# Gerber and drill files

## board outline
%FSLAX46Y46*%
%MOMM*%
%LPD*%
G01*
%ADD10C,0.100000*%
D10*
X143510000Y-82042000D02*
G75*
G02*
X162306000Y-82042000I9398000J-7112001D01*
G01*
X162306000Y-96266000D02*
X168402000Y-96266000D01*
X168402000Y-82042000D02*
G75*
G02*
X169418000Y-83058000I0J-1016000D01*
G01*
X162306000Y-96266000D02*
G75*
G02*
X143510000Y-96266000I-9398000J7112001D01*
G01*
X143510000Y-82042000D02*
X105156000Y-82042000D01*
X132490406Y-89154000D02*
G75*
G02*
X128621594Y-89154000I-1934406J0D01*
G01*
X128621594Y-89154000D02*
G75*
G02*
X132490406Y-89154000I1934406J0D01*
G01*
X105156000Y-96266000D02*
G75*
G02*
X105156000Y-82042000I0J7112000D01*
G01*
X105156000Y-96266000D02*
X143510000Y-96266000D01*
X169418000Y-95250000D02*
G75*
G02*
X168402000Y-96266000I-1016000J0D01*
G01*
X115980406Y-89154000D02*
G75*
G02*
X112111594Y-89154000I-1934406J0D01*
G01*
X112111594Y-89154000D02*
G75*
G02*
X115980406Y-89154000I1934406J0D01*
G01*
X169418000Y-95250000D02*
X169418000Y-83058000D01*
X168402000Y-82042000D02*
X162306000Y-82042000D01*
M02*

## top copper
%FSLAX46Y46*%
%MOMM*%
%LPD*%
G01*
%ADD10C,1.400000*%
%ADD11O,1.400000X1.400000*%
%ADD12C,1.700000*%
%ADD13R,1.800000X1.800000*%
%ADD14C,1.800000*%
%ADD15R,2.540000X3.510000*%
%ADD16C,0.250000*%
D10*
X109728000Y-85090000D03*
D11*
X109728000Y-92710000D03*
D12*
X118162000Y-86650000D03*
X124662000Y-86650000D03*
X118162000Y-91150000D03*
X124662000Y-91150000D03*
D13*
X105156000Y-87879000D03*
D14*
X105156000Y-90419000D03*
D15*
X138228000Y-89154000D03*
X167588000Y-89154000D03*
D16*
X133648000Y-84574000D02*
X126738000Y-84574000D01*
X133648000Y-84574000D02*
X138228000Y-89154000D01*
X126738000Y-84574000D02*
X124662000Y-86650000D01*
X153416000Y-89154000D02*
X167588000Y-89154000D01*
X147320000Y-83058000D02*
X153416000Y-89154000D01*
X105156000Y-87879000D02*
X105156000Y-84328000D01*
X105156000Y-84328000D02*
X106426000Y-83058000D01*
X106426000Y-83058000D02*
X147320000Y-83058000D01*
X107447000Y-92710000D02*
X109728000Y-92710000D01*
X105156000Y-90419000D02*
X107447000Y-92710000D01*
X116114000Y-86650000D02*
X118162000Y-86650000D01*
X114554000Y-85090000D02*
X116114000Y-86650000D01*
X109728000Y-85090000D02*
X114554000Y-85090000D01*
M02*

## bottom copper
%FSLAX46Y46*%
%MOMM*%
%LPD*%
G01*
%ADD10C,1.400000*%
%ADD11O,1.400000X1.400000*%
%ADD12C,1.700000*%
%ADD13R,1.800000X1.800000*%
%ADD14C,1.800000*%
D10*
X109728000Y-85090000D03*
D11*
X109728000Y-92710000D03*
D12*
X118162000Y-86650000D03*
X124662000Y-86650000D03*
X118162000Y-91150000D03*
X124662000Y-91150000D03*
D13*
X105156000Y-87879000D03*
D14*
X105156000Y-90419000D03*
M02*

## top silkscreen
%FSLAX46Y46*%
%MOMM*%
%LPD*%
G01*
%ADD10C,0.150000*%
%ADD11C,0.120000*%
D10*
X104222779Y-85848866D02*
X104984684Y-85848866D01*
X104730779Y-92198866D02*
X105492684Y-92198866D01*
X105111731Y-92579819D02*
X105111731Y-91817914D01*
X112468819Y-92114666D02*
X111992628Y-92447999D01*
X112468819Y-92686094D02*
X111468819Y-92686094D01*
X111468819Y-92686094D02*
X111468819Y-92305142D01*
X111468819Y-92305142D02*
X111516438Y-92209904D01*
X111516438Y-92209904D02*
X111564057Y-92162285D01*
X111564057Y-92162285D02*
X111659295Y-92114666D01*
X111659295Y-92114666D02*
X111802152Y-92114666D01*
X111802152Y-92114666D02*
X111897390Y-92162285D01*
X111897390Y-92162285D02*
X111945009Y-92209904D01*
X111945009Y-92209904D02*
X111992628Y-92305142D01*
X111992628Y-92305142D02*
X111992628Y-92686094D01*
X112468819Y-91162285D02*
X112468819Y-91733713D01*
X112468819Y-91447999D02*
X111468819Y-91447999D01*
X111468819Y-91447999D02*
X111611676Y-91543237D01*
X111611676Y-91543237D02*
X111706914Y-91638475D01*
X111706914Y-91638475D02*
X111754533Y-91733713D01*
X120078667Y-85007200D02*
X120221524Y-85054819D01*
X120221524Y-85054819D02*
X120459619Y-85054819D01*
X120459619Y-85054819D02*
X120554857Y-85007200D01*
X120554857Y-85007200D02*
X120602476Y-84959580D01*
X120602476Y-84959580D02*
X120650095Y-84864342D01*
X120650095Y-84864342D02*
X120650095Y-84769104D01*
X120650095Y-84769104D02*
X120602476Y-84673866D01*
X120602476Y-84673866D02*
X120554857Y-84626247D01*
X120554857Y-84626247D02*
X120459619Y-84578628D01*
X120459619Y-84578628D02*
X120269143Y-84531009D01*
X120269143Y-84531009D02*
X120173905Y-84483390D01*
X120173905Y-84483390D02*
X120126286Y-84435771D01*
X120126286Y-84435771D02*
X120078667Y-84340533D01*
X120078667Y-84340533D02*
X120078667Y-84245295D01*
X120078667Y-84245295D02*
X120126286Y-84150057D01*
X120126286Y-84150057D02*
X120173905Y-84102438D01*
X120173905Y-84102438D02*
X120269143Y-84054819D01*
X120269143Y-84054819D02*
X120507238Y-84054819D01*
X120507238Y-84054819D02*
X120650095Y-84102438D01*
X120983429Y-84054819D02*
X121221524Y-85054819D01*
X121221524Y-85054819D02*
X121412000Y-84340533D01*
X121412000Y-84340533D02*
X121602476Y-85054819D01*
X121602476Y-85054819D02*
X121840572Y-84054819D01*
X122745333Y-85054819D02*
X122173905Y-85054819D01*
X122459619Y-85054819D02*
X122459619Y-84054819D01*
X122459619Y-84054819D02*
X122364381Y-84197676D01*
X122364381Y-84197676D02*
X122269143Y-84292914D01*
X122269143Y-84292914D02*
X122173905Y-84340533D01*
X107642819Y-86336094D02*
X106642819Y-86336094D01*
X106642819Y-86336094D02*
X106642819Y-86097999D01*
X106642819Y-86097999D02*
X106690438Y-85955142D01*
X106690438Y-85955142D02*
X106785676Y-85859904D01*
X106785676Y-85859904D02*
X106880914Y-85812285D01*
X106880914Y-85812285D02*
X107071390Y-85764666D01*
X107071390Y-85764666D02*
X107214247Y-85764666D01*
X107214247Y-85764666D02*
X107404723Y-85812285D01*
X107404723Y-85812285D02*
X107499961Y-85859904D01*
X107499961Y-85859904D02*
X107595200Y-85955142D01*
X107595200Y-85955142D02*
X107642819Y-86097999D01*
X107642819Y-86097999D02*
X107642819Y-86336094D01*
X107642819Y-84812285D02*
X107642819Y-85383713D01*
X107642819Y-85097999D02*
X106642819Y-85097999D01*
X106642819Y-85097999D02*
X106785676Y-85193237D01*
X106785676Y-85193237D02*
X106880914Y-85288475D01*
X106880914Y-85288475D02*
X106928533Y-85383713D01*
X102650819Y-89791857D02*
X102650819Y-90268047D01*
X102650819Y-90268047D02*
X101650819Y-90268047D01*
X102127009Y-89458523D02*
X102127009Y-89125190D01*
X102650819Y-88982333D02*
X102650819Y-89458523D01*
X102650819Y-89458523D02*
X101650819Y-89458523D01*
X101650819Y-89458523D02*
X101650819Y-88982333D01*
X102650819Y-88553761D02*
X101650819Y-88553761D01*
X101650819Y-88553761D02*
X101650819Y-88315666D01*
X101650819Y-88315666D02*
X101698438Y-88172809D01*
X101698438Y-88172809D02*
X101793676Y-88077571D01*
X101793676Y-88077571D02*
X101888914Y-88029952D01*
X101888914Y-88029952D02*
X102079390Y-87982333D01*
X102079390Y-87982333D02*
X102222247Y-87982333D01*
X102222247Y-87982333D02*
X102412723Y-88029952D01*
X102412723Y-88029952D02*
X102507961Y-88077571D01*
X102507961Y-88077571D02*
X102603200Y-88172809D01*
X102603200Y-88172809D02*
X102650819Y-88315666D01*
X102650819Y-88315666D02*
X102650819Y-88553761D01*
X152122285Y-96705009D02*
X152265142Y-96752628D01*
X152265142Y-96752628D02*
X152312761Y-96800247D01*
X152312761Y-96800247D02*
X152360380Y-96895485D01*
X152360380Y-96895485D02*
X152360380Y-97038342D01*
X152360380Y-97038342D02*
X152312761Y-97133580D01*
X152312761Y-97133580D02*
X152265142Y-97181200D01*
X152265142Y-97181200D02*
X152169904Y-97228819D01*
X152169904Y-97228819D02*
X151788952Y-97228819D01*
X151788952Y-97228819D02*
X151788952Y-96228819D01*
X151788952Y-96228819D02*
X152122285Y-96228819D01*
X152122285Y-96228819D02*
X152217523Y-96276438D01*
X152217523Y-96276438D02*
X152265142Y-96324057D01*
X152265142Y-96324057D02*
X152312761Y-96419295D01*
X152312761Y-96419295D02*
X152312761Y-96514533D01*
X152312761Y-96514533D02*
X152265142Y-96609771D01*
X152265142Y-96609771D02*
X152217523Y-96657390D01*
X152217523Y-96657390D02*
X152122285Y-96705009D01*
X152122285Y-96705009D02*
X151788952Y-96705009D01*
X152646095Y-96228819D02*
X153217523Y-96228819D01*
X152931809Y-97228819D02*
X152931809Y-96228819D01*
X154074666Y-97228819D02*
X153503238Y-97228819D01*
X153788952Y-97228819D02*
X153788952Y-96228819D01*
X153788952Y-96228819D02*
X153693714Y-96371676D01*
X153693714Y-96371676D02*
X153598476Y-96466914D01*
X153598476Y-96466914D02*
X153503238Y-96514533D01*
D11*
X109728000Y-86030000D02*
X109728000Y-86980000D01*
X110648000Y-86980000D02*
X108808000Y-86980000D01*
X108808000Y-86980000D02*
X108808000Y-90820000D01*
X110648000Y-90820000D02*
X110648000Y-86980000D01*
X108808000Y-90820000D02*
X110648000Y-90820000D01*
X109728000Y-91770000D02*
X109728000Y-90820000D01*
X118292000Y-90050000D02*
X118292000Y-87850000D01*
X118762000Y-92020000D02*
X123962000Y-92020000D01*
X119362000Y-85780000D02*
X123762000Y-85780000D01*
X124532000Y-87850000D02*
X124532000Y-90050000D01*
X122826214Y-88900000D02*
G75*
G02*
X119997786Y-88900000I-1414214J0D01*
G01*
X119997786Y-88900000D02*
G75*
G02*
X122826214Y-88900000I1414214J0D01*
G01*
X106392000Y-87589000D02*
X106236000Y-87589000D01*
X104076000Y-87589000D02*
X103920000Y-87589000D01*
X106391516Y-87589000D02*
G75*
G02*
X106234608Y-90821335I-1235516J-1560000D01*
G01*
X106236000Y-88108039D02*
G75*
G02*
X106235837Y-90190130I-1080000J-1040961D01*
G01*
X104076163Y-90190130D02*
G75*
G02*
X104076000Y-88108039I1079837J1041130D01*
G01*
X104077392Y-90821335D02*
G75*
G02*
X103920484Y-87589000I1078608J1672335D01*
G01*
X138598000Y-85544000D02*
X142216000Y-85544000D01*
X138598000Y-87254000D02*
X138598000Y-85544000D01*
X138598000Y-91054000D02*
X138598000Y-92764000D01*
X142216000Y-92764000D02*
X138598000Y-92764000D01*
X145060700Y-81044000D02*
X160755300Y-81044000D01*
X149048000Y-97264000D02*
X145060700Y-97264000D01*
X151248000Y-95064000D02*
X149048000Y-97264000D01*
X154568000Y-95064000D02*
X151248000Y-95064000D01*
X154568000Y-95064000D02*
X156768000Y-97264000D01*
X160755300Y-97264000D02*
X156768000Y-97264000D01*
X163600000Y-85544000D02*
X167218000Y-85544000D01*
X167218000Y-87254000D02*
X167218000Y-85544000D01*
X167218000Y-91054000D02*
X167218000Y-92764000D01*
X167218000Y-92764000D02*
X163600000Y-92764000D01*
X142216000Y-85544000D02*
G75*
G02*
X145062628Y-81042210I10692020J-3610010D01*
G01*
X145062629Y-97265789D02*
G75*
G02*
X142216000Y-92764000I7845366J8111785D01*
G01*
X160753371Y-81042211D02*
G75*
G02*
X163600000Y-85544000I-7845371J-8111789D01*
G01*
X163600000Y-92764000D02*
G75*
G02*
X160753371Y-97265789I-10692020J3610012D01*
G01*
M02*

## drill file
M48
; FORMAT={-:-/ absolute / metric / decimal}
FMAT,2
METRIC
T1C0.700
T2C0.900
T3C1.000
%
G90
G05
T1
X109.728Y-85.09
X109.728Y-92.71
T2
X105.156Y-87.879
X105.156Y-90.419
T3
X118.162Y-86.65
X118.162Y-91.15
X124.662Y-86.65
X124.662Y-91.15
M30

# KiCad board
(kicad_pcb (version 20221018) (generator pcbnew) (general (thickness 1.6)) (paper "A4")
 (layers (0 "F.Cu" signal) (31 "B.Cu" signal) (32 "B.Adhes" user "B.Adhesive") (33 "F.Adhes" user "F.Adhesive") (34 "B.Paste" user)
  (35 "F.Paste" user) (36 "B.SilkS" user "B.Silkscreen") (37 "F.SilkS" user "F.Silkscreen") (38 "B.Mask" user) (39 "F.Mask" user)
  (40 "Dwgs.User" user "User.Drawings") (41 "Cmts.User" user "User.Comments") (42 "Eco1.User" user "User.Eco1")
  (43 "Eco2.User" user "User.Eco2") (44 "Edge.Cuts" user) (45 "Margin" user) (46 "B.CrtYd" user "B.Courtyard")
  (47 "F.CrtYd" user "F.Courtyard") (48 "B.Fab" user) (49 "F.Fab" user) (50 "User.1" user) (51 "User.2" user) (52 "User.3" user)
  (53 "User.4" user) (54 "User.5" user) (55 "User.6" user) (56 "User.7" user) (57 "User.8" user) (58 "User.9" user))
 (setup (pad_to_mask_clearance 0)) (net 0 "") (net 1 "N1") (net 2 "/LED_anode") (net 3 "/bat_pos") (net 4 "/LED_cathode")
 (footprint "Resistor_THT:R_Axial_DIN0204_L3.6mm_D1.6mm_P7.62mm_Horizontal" (layer "F.Cu") (at 109.728 85.09 -90)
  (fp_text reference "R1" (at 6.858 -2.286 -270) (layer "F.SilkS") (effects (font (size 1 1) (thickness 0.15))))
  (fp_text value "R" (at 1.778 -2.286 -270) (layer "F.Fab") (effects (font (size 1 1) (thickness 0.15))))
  (fp_line (start 0.94 0) (end 1.89 0) (stroke (width 0.12) (type solid)) (layer "F.SilkS"))
  (fp_line (start 1.89 -0.92) (end 1.89 0.92) (stroke (width 0.12) (type solid)) (layer "F.SilkS"))
  (fp_line (start 1.89 0.92) (end 5.73 0.92) (stroke (width 0.12) (type solid)) (layer "F.SilkS"))
  (fp_line (start 5.73 -0.92) (end 1.89 -0.92) (stroke (width 0.12) (type solid)) (layer "F.SilkS"))
  (fp_line (start 5.73 0.92) (end 5.73 -0.92) (stroke (width 0.12) (type solid)) (layer "F.SilkS"))
  (fp_line (start 6.68 0) (end 5.73 0) (stroke (width 0.12) (type solid)) (layer "F.SilkS"))
  (pad "1" thru_hole circle (at 0 0 270) (size 1.4 1.4) (drill 0.7) (layers "*.Cu" "*.Mask") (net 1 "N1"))
  (pad "2" thru_hole oval (at 7.62 0 270) (size 1.4 1.4) (drill 0.7) (layers "*.Cu" "*.Mask") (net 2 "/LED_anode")))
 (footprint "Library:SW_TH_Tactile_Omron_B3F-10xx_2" (layer "F.Cu") (at 118.162 86.65)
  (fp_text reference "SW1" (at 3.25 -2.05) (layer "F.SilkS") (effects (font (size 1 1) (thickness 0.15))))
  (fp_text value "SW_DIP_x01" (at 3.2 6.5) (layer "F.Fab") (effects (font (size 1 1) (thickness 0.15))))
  (fp_line (start 0.13 3.4) (end 0.13 1.2) (stroke (width 0.12) (type solid)) (layer "F.SilkS"))
  (fp_line (start 0.6 5.37) (end 5.8 5.37) (stroke (width 0.12) (type solid)) (layer "F.SilkS"))
  (fp_line (start 1.2 -0.87) (end 5.6 -0.87) (stroke (width 0.12) (type solid)) (layer "F.SilkS"))
  (fp_line (start 6.37 1.2) (end 6.37 3.4) (stroke (width 0.12) (type solid)) (layer "F.SilkS"))
  (fp_circle (center 3.25 2.25) (end 4.25 3.25) (stroke (width 0.12) (type solid)) (fill none) (layer "F.SilkS"))
  (pad "1" thru_hole circle (at 0 0) (size 1.7 1.7) (drill 1) (layers "*.Cu" "*.Mask") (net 1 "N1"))
  (pad "2" thru_hole circle (at 6.5 0) (size 1.7 1.7) (drill 1) (layers "*.Cu" "*.Mask") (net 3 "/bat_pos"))
  (pad "3" thru_hole circle (at 0 4.5) (size 1.7 1.7) (drill 1) (layers "*.Cu" "*.Mask"))
  (pad "4" thru_hole circle (at 6.5 4.5) (size 1.7 1.7) (drill 1) (layers "*.Cu" "*.Mask")))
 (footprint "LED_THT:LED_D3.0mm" (layer "F.Cu") (at 105.156 87.879 -90)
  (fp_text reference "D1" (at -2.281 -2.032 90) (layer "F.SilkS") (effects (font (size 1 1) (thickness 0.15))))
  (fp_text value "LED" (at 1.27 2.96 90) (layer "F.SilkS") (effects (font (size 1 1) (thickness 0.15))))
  (fp_line (start -0.29 -1.236) (end -0.29 -1.08) (stroke (width 0.12) (type solid)) (layer "F.SilkS"))
  (fp_line (start -0.29 1.08) (end -0.29 1.236) (stroke (width 0.12) (type solid)) (layer "F.SilkS"))
  (fp_arc (start -0.29 -1.235516) (mid 1.366487 -1.987659) (end 2.942335 -1.078608) (stroke (width 0.12) (type solid)) (layer "F.SilkS"))
  (fp_arc (start 0.229039 -1.08) (mid 1.270117 -1.5) (end 2.31113 -1.079837) (stroke (width 0.12) (type solid)) (layer "F.SilkS"))
  (fp_arc (start 2.31113 1.079837) (mid 1.270117 1.5) (end 0.229039 1.08) (stroke (width 0.12) (type solid)) (layer "F.SilkS"))
  (fp_arc (start 2.942335 1.078608) (mid 1.366487 1.987659) (end -0.29 1.235516) (stroke (width 0.12) (type solid)) (layer "F.SilkS"))
  (pad "1" thru_hole rect (at 0 0 270) (size 1.8 1.8) (drill 0.9) (layers "*.Cu" "*.Mask") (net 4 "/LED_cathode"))
  (pad "2" thru_hole circle (at 2.54 0 270) (size 1.8 1.8) (drill 0.9) (layers "*.Cu" "*.Mask") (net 2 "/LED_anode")))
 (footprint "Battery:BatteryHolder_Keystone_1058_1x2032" (layer "F.Cu") (at 152.908 89.154)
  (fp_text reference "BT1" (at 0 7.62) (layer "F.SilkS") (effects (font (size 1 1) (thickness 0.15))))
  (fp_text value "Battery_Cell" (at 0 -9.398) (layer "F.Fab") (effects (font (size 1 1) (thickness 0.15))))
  (fp_line (start -14.31 -3.61) (end -10.692 -3.61) (stroke (width 0.12) (type solid)) (layer "F.SilkS"))
  (fp_line (start -14.31 -1.9) (end -14.31 -3.61) (stroke (width 0.12) (type solid)) (layer "F.SilkS"))
  (fp_line (start -14.31 1.9) (end -14.31 3.61) (stroke (width 0.12) (type solid)) (layer "F.SilkS"))
  (fp_line (start -10.692 3.61) (end -14.31 3.61) (stroke (width 0.12) (type solid)) (layer "F.SilkS"))
  (fp_line (start -7.8473 -8.11) (end 7.8473 -8.11) (stroke (width 0.12) (type solid)) (layer "F.SilkS"))
  (fp_line (start -3.86 8.11) (end -7.8473 8.11) (stroke (width 0.12) (type solid)) (layer "F.SilkS"))
  (fp_line (start -1.66 5.91) (end -3.86 8.11) (stroke (width 0.12) (type solid)) (layer "F.SilkS"))
  (fp_line (start 1.66 5.91) (end -1.66 5.91) (stroke (width 0.12) (type solid)) (layer "F.SilkS"))
  (fp_line (start 1.66 5.91) (end 3.86 8.11) (stroke (width 0.12) (type solid)) (layer "F.SilkS"))
  (fp_line (start 7.8473 8.11) (end 3.86 8.11) (stroke (width 0.12) (type solid)) (layer "F.SilkS"))
  (fp_line (start 10.692 -3.61) (end 14.31 -3.61) (stroke (width 0.12) (type solid)) (layer "F.SilkS"))
  (fp_line (start 14.31 -1.9) (end 14.31 -3.61) (stroke (width 0.12) (type solid)) (layer "F.SilkS"))
  (fp_line (start 14.31 1.9) (end 14.31 3.61) (stroke (width 0.12) (type solid)) (layer "F.SilkS"))
  (fp_line (start 14.31 3.61) (end 10.692 3.61) (stroke (width 0.12) (type solid)) (layer "F.SilkS"))
  (fp_arc (start -10.692 -3.61) (mid -9.538084 -6.031244) (end -7.845371 -8.111789) (stroke (width 0.12) (type solid)) (layer "F.SilkS"))
  (fp_arc (start -7.845371 8.111789) (mid -9.538085 6.031244) (end -10.692 3.61) (stroke (width 0.12) (type solid)) (layer "F.SilkS"))
  (fp_arc (start 7.845371 -8.111789) (mid 9.538085 -6.031244) (end 10.692 -3.61) (stroke (width 0.12) (type solid)) (layer "F.SilkS"))
  (fp_arc (start 10.692 3.61) (mid 9.538084 6.031244) (end 7.845371 8.111789) (stroke (width 0.12) (type solid)) (layer "F.SilkS"))
  (pad "1" smd rect (at -14.68 0) (size 2.54 3.51) (layers "F.Cu" "F.Paste" "F.Mask") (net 3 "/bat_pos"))
  (pad "2" smd rect (at 14.68 0) (size 2.54 3.51) (layers "F.Cu" "F.Paste" "F.Mask") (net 4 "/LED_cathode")))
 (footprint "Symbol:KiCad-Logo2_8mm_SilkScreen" (layer "B.Cu") (at 153.162 88.138 180)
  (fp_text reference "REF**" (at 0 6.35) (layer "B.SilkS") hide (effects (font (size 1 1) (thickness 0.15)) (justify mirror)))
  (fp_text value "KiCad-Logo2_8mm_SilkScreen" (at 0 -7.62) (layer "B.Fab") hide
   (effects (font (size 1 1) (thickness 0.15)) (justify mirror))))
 (gr_arc (start 143.51 82.042) (mid 152.908 77.368291) (end 162.306 82.042) (stroke (width 0.1) (type default)) (layer "Edge.Cuts"))
 (gr_line (start 162.306 96.266) (end 168.402 96.266) (stroke (width 0.1) (type default)) (layer "Edge.Cuts"))
 (gr_arc (start 168.402 82.042) (mid 169.12042 82.33958) (end 169.418 83.058) (stroke (width 0.1) (type default)) (layer "Edge.Cuts"))
 (gr_arc (start 162.306 96.266) (mid 152.908 100.939709) (end 143.51 96.266) (stroke (width 0.1) (type default)) (layer "Edge.Cuts"))
 (gr_line (start 143.51 82.042) (end 105.156 82.042) (stroke (width 0.1) (type default)) (layer "Edge.Cuts"))
 (gr_circle (center 130.556 89.154) (end 132.490406 89.154) (stroke (width 0.1) (type default)) (fill none) (layer "Edge.Cuts"))
 (gr_arc (start 105.156 96.266) (mid 98.044 89.154) (end 105.156 82.042) (stroke (width 0.1) (type default)) (layer "Edge.Cuts"))
 (gr_line (start 105.156 96.266) (end 143.51 96.266) (stroke (width 0.1) (type default)) (layer "Edge.Cuts"))
 (gr_arc (start 169.418 95.25) (mid 169.12042 95.96842) (end 168.402 96.266) (stroke (width 0.1) (type default)) (layer "Edge.Cuts"))
 (gr_circle (center 114.046 89.154) (end 115.980406 89.154) (stroke (width 0.1) (type default)) (fill none) (layer "Edge.Cuts"))
 (gr_line (start 169.418 95.25) (end 169.418 83.058) (stroke (width 0.1) (type default)) (layer "Edge.Cuts"))
 (gr_line (start 168.402 82.042) (end 162.306 82.042) (stroke (width 0.1) (type default)) (layer "Edge.Cuts"))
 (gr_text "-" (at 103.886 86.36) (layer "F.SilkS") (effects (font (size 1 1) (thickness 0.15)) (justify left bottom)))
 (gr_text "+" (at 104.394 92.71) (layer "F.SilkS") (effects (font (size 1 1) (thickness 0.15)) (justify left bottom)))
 (segment (start 133.648 84.574) (end 126.738 84.574) (width 0.25) (layer "F.Cu") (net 3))
 (segment (start 133.648 84.574) (end 138.228 89.154) (width 0.25) (layer "F.Cu") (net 3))
 (segment (start 126.738 84.574) (end 124.662 86.65) (width 0.25) (layer "F.Cu") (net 3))
 (segment (start 153.416 89.154) (end 167.588 89.154) (width 0.25) (layer "F.Cu") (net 4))
 (segment (start 147.32 83.058) (end 153.416 89.154) (width 0.25) (layer "F.Cu") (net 4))
 (segment (start 105.156 87.879) (end 105.156 84.328) (width 0.25) (layer "F.Cu") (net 4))
 (segment (start 105.156 84.328) (end 106.426 83.058) (width 0.25) (layer "F.Cu") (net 4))
 (segment (start 106.426 83.058) (end 147.32 83.058) (width 0.25) (layer "F.Cu") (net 4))
 (segment (start 107.447 92.71) (end 109.728 92.71) (width 0.25) (layer "F.Cu") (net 2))
 (segment (start 105.156 90.419) (end 107.447 92.71) (width 0.25) (layer "F.Cu") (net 2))
 (segment (start 116.114 86.65) (end 118.162 86.65) (width 0.25) (layer "F.Cu") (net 1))
 (segment (start 114.554 85.09) (end 116.114 86.65) (width 0.25) (layer "F.Cu") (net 1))
 (segment (start 109.728 85.09) (end 114.554 85.09) (width 0.25) (layer "F.Cu") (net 1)))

